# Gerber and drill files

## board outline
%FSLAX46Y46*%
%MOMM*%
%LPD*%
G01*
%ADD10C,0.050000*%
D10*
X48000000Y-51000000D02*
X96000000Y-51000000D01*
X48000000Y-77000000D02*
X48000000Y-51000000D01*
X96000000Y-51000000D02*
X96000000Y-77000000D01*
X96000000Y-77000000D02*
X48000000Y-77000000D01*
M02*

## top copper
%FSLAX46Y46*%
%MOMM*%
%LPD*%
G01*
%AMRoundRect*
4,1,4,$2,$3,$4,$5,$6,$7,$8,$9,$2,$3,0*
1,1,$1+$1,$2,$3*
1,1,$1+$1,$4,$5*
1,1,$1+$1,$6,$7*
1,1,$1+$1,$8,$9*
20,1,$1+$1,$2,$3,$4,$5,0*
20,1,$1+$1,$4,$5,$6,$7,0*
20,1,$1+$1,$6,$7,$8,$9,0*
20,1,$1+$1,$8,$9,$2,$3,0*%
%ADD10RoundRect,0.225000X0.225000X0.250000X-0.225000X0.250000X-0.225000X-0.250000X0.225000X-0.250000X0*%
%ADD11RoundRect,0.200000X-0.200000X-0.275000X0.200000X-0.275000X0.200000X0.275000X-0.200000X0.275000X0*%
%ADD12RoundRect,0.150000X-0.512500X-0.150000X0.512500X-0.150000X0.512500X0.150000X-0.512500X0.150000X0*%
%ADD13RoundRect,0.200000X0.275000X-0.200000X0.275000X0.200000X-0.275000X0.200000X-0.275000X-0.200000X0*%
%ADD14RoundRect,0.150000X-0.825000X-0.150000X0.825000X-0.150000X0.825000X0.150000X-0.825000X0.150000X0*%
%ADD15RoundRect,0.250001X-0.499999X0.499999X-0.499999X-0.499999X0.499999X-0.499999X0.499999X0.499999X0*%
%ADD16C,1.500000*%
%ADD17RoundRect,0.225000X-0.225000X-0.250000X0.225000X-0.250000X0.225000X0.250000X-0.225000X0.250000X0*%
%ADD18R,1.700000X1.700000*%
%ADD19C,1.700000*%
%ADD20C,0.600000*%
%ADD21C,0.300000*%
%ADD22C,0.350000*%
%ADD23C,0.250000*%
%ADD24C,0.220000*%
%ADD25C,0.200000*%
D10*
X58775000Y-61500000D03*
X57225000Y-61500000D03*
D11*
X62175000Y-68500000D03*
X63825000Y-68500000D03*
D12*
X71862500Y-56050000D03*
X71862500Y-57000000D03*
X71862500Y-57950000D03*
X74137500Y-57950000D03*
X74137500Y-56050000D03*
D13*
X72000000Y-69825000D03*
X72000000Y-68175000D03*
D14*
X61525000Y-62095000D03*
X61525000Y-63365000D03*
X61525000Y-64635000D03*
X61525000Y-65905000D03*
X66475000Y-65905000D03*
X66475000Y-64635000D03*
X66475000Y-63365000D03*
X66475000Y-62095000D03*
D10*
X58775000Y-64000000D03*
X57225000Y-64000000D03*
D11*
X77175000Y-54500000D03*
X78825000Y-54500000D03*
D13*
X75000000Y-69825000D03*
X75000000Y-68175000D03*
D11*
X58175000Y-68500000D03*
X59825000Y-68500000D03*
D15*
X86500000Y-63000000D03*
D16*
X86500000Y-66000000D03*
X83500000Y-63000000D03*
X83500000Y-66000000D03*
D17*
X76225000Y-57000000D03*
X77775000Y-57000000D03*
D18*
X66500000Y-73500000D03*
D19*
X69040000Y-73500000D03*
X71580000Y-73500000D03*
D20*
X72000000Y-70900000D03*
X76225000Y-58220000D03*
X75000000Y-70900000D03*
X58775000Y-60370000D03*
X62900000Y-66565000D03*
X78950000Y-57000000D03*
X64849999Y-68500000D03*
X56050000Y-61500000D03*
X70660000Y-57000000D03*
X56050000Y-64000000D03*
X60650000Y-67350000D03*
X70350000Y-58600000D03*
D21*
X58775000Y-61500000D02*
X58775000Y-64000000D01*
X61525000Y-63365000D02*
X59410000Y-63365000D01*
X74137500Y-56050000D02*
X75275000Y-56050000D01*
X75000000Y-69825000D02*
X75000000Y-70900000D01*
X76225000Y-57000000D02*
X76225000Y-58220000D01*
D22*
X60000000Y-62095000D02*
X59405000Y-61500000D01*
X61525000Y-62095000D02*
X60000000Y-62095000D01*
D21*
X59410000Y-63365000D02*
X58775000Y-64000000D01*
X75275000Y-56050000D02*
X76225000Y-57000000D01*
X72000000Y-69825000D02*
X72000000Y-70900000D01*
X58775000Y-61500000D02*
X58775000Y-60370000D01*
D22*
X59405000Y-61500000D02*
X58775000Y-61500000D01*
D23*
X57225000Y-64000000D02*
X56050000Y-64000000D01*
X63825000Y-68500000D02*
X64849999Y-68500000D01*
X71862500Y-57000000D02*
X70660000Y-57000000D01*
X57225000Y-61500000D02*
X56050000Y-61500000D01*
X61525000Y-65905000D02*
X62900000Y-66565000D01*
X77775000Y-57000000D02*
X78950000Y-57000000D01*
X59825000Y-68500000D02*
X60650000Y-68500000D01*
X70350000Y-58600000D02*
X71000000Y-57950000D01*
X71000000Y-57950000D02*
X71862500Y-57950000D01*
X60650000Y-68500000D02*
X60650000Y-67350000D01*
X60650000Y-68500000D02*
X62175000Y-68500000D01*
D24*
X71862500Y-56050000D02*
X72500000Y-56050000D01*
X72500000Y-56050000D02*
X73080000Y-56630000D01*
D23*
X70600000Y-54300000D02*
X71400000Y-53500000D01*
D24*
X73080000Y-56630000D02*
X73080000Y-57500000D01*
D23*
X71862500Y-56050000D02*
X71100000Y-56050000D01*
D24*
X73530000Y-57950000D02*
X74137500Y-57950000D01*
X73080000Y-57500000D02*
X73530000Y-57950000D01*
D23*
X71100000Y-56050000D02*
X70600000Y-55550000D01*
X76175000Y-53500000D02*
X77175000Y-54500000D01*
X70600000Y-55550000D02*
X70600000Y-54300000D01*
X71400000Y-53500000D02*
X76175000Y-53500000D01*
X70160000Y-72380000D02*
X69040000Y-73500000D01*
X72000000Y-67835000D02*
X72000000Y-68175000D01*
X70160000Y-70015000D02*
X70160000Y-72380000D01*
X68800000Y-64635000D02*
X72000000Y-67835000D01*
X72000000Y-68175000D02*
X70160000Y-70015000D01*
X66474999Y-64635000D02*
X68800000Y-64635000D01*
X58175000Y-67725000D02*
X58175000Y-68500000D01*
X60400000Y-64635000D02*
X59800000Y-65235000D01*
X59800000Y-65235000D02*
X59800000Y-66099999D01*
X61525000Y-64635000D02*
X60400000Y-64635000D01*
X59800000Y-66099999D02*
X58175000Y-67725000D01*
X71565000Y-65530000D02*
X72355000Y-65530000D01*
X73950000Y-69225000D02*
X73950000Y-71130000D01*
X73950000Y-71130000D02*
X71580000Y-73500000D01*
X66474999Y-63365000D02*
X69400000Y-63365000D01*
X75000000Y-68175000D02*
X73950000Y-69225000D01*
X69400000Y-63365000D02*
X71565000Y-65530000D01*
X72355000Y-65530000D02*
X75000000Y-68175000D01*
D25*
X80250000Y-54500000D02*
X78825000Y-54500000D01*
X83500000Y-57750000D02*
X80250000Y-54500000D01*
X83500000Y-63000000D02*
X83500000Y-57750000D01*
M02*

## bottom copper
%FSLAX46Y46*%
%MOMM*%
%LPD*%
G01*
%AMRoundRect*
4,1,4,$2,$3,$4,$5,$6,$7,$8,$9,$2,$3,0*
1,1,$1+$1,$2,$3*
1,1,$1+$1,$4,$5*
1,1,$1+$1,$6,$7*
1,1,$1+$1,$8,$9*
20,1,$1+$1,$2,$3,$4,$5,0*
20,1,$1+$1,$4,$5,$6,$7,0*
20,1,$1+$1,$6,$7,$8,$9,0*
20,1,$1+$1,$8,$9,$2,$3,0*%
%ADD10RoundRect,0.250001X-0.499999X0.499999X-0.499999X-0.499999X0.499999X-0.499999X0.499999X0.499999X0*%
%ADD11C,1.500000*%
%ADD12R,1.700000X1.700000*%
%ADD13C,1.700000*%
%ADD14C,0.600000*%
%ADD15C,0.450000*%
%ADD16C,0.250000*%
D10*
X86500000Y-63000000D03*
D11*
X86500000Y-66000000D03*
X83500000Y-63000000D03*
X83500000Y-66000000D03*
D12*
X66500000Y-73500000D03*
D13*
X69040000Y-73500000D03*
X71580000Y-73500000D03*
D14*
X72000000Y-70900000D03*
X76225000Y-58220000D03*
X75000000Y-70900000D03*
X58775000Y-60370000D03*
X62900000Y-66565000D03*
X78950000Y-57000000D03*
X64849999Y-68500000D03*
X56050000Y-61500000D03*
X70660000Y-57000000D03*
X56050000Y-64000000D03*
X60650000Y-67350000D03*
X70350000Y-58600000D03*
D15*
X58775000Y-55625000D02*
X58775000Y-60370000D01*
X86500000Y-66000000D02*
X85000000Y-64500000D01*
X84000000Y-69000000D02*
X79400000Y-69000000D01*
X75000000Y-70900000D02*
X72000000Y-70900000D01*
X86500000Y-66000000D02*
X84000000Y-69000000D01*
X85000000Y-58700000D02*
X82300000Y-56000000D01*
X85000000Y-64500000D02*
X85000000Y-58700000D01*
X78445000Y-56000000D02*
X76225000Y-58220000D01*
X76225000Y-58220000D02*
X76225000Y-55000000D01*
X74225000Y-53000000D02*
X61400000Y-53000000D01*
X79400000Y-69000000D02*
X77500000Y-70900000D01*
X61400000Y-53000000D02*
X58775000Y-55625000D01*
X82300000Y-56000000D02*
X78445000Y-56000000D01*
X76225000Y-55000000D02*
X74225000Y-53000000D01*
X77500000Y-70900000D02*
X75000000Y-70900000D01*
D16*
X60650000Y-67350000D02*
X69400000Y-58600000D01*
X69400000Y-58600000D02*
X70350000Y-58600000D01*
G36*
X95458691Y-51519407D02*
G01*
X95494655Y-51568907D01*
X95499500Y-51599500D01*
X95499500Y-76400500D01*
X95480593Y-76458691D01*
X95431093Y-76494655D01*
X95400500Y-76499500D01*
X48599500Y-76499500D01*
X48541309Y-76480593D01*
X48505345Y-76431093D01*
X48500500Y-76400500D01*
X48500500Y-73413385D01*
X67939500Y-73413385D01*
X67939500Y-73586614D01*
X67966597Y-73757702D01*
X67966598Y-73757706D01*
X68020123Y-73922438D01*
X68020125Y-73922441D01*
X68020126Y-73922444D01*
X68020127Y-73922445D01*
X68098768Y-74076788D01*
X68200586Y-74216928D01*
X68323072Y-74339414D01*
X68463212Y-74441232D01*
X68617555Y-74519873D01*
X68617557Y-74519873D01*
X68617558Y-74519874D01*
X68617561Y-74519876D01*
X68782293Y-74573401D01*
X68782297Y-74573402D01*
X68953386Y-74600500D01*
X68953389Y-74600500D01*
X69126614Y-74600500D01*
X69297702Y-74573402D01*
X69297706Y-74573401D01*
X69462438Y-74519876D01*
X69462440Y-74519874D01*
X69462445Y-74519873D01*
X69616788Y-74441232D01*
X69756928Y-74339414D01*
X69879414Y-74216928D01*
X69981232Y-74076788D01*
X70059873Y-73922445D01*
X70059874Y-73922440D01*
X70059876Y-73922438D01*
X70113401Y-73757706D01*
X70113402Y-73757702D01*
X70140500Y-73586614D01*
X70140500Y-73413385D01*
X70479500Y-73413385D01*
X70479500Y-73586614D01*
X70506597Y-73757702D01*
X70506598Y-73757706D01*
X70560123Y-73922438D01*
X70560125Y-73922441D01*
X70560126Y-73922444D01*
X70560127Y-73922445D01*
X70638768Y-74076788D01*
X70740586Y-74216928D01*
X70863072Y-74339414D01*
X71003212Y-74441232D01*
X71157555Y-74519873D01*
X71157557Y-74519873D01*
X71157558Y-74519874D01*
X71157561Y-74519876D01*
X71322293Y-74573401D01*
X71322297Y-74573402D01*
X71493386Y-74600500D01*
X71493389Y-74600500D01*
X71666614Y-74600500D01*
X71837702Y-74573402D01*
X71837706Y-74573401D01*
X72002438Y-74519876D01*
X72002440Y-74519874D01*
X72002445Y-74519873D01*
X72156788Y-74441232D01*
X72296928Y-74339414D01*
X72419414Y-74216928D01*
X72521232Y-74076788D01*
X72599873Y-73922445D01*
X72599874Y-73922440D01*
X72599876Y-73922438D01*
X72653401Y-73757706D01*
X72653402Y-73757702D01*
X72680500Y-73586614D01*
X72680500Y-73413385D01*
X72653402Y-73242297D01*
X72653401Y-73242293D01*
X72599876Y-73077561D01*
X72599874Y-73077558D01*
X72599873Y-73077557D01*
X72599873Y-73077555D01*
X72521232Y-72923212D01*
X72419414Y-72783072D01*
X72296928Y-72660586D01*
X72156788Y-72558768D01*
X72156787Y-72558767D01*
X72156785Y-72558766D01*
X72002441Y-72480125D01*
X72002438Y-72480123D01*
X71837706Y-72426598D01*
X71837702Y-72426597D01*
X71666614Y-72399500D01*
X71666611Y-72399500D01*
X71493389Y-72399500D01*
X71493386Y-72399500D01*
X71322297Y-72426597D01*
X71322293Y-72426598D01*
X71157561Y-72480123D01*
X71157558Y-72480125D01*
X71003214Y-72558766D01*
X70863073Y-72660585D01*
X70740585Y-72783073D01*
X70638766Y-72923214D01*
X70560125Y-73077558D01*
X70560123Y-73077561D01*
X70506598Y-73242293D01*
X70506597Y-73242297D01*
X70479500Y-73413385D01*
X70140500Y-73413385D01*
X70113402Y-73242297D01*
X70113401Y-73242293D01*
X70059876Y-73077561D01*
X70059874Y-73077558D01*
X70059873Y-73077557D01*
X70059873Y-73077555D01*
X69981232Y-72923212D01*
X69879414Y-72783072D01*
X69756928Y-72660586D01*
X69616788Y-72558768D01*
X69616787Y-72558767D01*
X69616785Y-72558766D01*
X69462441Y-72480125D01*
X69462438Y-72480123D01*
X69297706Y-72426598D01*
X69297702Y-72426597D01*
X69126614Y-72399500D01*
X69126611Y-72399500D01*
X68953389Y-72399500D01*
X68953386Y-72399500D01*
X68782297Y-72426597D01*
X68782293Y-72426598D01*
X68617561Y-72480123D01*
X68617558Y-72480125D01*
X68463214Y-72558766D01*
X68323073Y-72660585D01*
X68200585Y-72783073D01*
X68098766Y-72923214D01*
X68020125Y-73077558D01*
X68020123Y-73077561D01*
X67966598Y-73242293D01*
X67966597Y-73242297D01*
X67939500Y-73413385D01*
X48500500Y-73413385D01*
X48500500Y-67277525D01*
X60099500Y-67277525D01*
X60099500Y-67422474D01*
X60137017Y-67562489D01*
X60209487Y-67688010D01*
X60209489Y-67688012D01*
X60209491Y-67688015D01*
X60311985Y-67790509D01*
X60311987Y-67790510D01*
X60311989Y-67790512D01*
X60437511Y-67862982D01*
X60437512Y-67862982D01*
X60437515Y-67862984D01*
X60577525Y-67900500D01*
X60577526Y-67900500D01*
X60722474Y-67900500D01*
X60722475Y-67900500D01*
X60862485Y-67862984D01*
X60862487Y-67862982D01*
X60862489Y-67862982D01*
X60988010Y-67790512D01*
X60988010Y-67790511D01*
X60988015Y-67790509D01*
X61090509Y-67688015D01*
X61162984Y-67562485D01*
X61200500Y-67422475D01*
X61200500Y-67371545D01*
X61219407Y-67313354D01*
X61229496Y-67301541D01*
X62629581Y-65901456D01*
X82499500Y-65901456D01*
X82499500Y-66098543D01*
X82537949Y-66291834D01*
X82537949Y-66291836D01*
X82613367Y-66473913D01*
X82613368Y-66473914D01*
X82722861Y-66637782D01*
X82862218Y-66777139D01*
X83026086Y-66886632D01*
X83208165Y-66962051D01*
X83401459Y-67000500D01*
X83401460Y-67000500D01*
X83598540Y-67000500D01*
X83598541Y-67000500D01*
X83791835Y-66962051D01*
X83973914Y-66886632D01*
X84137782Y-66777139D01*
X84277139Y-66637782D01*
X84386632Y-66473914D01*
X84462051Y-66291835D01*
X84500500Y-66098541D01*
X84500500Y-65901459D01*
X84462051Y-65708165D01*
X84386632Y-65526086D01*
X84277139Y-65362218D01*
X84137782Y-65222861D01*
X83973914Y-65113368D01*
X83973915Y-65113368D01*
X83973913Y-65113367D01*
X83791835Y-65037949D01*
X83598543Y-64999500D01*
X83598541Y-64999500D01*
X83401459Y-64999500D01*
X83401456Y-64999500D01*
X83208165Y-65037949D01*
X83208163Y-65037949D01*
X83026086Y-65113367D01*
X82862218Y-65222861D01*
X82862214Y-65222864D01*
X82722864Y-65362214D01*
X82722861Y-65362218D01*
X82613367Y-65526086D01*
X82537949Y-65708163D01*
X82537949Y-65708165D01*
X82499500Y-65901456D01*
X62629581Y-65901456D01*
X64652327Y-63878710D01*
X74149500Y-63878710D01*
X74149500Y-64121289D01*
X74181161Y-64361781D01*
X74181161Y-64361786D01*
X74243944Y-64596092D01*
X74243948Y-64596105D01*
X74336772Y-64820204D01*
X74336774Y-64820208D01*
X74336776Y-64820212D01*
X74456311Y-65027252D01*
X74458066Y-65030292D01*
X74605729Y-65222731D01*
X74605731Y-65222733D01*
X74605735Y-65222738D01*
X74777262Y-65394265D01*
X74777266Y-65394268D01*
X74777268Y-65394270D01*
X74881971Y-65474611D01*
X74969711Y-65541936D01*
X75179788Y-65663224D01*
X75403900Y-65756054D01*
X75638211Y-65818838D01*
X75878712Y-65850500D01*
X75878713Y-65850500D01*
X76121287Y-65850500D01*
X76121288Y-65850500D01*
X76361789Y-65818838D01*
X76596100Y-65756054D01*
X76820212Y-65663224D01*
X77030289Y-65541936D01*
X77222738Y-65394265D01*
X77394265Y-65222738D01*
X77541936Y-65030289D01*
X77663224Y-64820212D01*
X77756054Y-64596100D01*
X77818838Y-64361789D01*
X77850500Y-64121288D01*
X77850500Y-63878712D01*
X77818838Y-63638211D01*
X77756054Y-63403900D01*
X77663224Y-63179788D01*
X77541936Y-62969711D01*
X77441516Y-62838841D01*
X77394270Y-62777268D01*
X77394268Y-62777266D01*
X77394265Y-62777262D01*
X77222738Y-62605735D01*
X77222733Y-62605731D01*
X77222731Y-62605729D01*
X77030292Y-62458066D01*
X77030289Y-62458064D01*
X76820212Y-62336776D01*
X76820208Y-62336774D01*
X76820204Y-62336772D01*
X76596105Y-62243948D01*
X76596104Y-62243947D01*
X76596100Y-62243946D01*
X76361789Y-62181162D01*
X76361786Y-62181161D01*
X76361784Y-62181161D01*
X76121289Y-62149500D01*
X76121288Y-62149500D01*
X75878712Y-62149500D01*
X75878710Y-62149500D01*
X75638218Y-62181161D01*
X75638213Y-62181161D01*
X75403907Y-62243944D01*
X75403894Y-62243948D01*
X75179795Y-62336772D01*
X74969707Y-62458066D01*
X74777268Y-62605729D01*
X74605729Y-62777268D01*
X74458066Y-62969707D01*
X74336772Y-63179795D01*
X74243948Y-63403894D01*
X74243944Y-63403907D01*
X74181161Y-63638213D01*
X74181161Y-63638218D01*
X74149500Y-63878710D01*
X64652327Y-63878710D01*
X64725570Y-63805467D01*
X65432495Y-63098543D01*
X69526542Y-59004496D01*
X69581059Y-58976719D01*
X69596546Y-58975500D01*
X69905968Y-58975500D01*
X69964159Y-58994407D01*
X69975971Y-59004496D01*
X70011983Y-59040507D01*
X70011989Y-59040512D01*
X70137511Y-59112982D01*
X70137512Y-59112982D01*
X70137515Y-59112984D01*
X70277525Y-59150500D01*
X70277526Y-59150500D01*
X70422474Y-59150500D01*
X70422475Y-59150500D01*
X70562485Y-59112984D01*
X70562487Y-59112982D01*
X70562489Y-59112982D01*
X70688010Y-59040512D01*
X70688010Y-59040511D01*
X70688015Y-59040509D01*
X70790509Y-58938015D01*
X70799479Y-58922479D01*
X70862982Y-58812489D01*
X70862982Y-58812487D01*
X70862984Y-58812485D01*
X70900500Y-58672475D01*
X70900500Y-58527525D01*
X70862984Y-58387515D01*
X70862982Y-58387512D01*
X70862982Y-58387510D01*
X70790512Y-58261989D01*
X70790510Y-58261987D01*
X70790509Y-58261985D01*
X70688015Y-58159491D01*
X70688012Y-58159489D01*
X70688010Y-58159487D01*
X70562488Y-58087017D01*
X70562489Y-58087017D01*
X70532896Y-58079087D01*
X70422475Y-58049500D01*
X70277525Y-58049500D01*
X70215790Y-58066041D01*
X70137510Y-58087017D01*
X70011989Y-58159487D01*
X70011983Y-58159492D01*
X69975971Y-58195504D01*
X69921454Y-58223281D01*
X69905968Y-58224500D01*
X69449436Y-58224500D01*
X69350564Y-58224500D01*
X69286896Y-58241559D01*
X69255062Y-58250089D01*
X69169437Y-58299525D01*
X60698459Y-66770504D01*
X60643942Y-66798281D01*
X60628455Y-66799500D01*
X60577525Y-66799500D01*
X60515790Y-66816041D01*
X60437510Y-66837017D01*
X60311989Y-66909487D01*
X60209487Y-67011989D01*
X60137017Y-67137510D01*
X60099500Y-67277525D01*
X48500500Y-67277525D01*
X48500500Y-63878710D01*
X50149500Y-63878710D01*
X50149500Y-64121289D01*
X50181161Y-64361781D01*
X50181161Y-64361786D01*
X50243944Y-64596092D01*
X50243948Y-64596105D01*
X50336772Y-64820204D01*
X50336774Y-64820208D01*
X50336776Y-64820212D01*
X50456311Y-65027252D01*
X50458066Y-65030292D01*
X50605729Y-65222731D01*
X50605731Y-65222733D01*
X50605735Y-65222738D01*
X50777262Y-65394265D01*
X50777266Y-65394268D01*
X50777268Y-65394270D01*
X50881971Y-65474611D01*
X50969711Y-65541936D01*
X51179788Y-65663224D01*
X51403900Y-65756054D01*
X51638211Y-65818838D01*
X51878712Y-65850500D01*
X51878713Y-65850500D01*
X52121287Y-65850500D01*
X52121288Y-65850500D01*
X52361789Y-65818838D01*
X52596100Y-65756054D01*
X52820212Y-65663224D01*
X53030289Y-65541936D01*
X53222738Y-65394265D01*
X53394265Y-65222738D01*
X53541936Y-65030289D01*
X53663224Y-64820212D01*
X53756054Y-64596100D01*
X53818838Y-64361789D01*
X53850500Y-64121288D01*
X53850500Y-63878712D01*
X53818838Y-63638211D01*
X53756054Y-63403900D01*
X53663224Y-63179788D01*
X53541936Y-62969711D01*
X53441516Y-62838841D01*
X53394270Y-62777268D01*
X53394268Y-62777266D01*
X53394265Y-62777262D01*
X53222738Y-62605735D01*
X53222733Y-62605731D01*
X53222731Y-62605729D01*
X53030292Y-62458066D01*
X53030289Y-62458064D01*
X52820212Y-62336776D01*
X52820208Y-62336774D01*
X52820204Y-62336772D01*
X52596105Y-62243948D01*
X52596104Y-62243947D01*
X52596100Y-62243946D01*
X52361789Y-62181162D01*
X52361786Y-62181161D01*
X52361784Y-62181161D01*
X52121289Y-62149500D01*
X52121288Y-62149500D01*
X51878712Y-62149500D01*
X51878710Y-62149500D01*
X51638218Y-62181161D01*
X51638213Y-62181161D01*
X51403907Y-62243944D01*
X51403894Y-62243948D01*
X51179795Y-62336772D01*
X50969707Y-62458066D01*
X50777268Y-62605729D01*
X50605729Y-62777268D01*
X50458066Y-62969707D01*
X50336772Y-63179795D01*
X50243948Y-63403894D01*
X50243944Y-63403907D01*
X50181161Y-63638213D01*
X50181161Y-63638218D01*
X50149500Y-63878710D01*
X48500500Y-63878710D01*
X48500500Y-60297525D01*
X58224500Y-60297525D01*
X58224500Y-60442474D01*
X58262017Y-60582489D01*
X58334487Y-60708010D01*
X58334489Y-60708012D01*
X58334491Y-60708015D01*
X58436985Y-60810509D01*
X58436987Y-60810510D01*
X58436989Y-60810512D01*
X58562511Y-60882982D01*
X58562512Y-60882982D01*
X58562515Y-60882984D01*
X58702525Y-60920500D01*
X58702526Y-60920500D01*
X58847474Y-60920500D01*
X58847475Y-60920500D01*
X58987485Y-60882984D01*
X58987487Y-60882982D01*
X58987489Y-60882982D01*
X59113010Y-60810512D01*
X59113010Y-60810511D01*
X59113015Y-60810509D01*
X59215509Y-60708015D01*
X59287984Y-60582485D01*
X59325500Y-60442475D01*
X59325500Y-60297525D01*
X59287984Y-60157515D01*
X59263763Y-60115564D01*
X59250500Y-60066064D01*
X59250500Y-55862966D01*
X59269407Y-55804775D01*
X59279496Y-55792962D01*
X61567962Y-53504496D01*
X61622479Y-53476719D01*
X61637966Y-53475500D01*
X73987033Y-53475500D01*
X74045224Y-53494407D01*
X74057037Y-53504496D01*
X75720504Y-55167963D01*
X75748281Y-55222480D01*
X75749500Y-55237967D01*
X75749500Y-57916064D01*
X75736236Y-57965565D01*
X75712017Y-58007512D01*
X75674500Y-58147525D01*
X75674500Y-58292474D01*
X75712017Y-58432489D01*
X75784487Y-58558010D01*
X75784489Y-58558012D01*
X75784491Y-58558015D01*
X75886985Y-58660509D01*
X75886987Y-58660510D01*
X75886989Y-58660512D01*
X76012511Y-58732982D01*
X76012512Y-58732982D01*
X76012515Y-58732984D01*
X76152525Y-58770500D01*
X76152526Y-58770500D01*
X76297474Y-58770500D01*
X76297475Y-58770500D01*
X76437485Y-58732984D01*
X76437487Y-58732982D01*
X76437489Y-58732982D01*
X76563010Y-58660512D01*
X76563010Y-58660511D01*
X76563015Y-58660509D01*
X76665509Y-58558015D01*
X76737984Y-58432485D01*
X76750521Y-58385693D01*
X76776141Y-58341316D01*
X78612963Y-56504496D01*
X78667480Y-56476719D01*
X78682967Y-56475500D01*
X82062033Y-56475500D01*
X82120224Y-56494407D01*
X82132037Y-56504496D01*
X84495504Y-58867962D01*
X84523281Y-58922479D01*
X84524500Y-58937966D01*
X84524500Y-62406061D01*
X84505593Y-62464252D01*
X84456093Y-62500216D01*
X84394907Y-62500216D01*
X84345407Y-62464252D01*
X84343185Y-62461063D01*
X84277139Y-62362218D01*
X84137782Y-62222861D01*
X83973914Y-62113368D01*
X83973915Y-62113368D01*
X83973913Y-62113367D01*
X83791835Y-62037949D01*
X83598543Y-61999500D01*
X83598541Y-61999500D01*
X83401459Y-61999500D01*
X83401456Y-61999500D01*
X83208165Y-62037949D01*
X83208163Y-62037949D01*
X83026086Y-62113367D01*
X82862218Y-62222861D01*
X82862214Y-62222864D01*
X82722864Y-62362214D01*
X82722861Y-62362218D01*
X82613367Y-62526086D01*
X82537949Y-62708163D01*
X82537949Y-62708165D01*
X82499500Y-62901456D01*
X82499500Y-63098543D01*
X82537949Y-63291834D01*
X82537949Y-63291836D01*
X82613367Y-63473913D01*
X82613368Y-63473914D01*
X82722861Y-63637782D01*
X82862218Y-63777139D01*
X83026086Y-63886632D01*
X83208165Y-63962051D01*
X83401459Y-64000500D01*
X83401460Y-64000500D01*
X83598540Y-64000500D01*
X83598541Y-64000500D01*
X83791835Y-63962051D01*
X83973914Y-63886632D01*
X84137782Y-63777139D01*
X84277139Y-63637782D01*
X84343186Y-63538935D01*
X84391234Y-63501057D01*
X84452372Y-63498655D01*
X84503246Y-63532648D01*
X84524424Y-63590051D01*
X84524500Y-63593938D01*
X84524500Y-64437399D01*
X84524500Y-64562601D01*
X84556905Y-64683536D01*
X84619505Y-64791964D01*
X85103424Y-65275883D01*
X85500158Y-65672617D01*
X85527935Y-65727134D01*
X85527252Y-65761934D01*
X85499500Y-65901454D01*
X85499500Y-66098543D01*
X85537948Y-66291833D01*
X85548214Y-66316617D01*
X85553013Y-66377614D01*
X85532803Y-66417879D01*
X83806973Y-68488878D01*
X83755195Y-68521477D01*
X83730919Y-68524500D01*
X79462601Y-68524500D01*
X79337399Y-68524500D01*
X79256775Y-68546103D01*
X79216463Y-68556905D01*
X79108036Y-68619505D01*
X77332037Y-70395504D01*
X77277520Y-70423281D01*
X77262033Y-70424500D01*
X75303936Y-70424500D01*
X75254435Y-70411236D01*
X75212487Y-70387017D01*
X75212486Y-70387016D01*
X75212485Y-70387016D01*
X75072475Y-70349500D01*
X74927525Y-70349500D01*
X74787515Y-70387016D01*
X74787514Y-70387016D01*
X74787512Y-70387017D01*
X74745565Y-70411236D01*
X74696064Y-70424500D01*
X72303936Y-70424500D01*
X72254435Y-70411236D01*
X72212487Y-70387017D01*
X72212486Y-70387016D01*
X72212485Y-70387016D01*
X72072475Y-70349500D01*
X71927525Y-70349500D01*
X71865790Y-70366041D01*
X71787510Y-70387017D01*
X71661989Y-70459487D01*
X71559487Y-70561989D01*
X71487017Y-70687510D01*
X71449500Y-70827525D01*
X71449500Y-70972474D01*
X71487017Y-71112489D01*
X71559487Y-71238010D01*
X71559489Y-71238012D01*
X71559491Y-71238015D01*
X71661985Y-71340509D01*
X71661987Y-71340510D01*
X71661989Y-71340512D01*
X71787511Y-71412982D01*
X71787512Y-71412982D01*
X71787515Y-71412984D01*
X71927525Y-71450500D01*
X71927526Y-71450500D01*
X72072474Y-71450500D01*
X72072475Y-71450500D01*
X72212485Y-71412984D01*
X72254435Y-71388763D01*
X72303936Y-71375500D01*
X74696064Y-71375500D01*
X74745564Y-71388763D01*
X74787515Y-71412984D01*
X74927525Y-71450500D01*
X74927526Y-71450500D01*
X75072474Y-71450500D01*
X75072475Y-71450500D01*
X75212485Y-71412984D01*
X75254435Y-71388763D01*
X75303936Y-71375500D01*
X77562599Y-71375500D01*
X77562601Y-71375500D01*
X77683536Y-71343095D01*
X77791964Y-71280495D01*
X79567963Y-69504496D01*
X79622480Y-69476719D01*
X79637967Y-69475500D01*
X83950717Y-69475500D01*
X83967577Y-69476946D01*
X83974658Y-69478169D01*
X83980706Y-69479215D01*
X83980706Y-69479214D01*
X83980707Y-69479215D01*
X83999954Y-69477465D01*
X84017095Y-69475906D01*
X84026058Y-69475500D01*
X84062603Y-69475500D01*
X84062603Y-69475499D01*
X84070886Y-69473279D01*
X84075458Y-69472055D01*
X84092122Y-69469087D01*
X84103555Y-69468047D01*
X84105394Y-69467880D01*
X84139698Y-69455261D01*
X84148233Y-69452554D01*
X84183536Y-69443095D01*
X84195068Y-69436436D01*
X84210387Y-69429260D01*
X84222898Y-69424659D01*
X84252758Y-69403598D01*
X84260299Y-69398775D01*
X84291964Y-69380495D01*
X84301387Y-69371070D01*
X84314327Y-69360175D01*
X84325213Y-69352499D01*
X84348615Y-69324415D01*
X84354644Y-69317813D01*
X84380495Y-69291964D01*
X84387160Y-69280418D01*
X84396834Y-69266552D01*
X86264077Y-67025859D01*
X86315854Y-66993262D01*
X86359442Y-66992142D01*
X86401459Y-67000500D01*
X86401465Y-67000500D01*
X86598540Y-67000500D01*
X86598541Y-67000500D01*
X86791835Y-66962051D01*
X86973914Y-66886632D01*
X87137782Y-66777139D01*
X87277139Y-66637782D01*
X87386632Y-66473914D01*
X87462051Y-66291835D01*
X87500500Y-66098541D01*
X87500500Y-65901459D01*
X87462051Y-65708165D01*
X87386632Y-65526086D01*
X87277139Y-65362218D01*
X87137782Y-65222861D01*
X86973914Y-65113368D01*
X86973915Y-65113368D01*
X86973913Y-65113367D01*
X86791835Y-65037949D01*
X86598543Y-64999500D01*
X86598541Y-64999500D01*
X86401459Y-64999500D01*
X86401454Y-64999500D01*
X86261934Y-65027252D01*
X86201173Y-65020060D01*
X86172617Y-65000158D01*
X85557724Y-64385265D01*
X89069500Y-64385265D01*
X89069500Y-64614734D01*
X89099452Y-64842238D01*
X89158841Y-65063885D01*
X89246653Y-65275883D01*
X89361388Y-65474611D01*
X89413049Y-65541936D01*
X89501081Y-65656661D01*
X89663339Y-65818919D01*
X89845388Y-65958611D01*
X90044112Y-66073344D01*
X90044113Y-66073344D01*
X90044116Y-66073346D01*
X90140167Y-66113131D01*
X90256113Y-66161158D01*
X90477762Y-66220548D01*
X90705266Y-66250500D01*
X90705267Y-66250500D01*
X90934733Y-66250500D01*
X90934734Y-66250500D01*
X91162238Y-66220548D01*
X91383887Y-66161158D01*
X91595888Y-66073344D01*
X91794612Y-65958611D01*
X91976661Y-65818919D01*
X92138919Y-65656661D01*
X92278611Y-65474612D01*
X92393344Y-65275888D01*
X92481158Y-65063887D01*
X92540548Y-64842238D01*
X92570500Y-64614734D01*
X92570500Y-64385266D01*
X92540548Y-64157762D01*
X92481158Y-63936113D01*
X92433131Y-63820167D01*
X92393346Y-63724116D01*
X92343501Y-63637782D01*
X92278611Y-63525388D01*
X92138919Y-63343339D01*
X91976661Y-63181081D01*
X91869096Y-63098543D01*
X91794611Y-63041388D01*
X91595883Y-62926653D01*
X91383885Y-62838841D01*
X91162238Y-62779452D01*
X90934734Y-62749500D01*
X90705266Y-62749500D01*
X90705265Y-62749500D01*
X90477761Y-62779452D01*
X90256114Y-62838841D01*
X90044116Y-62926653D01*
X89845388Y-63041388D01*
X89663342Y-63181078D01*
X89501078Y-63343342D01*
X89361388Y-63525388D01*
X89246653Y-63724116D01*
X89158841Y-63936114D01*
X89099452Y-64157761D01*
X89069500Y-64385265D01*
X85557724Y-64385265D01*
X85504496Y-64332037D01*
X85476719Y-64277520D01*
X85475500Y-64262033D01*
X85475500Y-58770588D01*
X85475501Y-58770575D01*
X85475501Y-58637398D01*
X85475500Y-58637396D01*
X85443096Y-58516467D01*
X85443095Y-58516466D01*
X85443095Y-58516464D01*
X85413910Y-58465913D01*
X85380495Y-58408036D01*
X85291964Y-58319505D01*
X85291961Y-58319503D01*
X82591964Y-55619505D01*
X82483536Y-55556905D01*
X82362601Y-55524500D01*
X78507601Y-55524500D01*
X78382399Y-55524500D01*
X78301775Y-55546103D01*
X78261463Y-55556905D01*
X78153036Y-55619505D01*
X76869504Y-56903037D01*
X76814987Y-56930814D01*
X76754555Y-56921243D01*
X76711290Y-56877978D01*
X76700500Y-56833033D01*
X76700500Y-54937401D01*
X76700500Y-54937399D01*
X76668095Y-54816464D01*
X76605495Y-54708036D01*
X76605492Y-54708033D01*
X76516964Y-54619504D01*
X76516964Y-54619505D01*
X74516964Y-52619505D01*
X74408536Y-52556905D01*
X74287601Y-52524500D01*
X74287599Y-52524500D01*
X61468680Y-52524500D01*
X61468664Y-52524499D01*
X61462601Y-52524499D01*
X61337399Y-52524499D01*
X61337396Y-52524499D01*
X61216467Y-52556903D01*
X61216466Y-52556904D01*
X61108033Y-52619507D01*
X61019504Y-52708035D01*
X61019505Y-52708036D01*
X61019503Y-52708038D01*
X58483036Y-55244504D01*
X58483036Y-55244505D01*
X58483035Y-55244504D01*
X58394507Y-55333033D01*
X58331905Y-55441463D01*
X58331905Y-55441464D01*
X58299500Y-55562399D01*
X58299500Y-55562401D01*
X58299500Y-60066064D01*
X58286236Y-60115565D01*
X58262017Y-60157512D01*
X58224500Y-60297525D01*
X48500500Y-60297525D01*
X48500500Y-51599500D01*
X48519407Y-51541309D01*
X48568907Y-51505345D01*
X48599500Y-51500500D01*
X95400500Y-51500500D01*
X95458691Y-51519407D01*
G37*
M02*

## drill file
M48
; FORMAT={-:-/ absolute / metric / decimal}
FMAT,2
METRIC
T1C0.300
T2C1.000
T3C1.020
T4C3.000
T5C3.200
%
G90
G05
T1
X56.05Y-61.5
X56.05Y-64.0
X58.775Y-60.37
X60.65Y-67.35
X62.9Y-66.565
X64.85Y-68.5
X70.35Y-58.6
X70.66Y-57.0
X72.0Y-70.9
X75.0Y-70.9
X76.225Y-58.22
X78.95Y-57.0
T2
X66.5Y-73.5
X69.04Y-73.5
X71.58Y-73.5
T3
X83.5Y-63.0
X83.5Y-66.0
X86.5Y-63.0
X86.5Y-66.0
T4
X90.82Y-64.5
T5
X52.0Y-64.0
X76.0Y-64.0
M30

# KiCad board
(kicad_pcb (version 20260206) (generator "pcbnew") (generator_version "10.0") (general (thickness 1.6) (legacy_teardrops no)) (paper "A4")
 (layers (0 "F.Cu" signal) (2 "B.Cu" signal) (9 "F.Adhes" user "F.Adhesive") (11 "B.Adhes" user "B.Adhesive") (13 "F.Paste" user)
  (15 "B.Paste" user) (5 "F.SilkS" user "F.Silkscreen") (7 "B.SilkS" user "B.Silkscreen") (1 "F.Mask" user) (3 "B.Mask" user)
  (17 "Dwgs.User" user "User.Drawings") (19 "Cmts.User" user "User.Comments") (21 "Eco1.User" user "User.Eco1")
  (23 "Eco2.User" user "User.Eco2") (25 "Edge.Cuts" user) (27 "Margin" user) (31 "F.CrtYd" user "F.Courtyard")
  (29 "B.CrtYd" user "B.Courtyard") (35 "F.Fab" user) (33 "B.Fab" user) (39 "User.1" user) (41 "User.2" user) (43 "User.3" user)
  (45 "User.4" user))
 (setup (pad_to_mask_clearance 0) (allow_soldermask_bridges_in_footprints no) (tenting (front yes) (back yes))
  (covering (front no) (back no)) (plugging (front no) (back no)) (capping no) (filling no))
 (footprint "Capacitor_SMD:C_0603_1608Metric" (layer "F.Cu") (at 58 61.5 180)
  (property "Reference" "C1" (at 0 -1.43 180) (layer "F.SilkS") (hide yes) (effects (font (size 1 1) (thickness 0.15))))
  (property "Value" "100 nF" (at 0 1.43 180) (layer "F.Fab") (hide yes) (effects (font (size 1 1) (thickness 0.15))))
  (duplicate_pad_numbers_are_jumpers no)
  (pad "1" smd roundrect (at -0.775 0 180) (size 0.9 0.95) (layers "F.Cu" "F.Mask" "F.Paste") (roundrect_rratio 0.25) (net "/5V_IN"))
  (pad "2" smd roundrect (at 0.775 0 180) (size 0.9 0.95) (layers "F.Cu" "F.Mask" "F.Paste") (roundrect_rratio 0.25) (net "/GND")))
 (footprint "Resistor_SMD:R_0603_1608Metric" (layer "F.Cu") (at 63 68.5)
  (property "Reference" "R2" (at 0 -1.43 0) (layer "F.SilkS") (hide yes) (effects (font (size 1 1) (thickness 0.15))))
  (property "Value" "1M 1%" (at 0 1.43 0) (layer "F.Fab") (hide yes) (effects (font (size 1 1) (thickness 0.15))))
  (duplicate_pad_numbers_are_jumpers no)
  (pad "1" smd roundrect (at -0.825 0) (size 0.8 0.95) (layers "F.Cu" "F.Mask" "F.Paste") (roundrect_rratio 0.25) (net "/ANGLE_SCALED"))
  (pad "2" smd roundrect (at 0.825 0) (size 0.8 0.95) (layers "F.Cu" "F.Mask" "F.Paste") (roundrect_rratio 0.25) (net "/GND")))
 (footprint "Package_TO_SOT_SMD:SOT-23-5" (layer "F.Cu") (at 73 57)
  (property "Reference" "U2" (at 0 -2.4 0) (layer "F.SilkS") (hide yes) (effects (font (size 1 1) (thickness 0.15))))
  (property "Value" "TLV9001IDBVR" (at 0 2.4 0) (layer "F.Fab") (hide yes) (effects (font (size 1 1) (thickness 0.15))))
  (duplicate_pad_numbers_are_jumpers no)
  (pad "1" smd roundrect (at -1.1375 -0.95) (size 1.325 0.6) (layers "F.Cu" "F.Mask" "F.Paste") (roundrect_rratio 0.25) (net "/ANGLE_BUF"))
  (pad "2" smd roundrect (at -1.1375 0) (size 1.325 0.6) (layers "F.Cu" "F.Mask" "F.Paste") (roundrect_rratio 0.25) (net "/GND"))
  (pad "3" smd roundrect (at -1.1375 0.95) (size 1.325 0.6) (layers "F.Cu" "F.Mask" "F.Paste") (roundrect_rratio 0.25) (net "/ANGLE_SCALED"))
  (pad "4" smd roundrect (at 1.1375 0.95) (size 1.325 0.6) (layers "F.Cu" "F.Mask" "F.Paste") (roundrect_rratio 0.25) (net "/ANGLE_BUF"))
  (pad "5" smd roundrect (at 1.1375 -0.95) (size 1.325 0.6) (layers "F.Cu" "F.Mask" "F.Paste") (roundrect_rratio 0.25) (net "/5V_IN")))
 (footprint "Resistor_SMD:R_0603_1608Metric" (layer "F.Cu") (at 72 69 90)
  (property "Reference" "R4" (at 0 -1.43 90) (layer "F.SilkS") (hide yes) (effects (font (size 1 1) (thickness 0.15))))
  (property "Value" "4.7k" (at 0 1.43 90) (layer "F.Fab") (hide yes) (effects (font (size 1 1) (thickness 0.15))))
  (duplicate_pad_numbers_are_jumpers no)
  (pad "1" smd roundrect (at -0.825 0 90) (size 0.8 0.95) (layers "F.Cu" "F.Mask" "F.Paste") (roundrect_rratio 0.25) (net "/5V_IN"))
  (pad "2" smd roundrect (at 0.825 0 90) (size 0.8 0.95) (layers "F.Cu" "F.Mask" "F.Paste") (roundrect_rratio 0.25) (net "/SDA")))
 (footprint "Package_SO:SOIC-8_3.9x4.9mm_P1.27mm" (layer "F.Cu") (at 64 64)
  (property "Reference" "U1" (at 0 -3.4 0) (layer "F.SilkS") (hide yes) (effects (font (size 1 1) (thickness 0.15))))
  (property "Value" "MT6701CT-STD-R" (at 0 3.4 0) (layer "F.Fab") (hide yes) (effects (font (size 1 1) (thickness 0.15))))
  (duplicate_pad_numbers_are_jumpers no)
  (pad "1" smd roundrect (at -2.475 -1.905) (size 1.95 0.6) (layers "F.Cu" "F.Mask" "F.Paste") (roundrect_rratio 0.25) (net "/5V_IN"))
  (pad "2" smd roundrect (at -2.475 -0.635) (size 1.95 0.6) (layers "F.Cu" "F.Mask" "F.Paste") (roundrect_rratio 0.25) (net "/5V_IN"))
  (pad "3" smd roundrect (at -2.475 0.635) (size 1.95 0.6) (layers "F.Cu" "F.Mask" "F.Paste") (roundrect_rratio 0.25) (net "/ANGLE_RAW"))
  (pad "4" smd roundrect (at -2.475 1.905) (size 1.95 0.6) (layers "F.Cu" "F.Mask" "F.Paste") (roundrect_rratio 0.25) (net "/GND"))
  (pad "5" smd roundrect (at 2.475 1.905) (size 1.95 0.6) (layers "F.Cu" "F.Mask" "F.Paste") (roundrect_rratio 0.25)
   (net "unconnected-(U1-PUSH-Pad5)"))
  (pad "6" smd roundrect (at 2.475 0.635) (size 1.95 0.6) (layers "F.Cu" "F.Mask" "F.Paste") (roundrect_rratio 0.25) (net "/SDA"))
  (pad "7" smd roundrect (at 2.475 -0.635) (size 1.95 0.6) (layers "F.Cu" "F.Mask" "F.Paste") (roundrect_rratio 0.25) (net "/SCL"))
  (pad "8" smd roundrect (at 2.475 -1.905) (size 1.95 0.6) (layers "F.Cu" "F.Mask" "F.Paste") (roundrect_rratio 0.25)
   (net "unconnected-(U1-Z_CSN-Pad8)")))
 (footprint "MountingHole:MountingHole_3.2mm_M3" (layer "F.Cu") (at 52 64)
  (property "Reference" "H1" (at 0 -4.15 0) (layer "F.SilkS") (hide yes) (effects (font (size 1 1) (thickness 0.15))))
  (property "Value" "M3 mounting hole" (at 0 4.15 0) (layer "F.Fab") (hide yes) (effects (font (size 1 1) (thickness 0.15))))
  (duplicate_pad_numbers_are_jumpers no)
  (pad "" np_thru_hole circle (at 0 0) (size 3.2 3.2) (drill 3.2) (layers "*.Cu" "*.Mask")))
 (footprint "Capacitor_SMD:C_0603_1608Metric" (layer "F.Cu") (at 58 64 180)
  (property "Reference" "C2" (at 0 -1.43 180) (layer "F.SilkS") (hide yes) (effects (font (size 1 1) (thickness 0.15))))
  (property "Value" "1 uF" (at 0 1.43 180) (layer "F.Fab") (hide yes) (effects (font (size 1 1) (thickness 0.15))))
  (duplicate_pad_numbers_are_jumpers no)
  (pad "1" smd roundrect (at -0.775 0 180) (size 0.9 0.95) (layers "F.Cu" "F.Mask" "F.Paste") (roundrect_rratio 0.25) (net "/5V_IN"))
  (pad "2" smd roundrect (at 0.775 0 180) (size 0.9 0.95) (layers "F.Cu" "F.Mask" "F.Paste") (roundrect_rratio 0.25) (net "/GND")))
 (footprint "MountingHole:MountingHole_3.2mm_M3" (layer "F.Cu") (at 76 64)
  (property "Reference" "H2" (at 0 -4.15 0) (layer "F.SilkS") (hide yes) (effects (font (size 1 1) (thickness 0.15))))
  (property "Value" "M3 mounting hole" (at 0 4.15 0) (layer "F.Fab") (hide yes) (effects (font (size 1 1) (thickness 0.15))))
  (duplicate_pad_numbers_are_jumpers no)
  (pad "" np_thru_hole circle (at 0 0) (size 3.2 3.2) (drill 3.2) (layers "*.Cu" "*.Mask")))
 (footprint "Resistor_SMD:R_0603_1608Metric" (layer "F.Cu") (at 78 54.5)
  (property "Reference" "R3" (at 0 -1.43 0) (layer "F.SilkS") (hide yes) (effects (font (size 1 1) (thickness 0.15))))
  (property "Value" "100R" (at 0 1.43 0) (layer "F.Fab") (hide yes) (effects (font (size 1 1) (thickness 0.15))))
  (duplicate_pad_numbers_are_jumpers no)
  (pad "1" smd roundrect (at -0.825 0) (size 0.8 0.95) (layers "F.Cu" "F.Mask" "F.Paste") (roundrect_rratio 0.25) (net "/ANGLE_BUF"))
  (pad "2" smd roundrect (at 0.825 0) (size 0.8 0.95) (layers "F.Cu" "F.Mask" "F.Paste") (roundrect_rratio 0.25) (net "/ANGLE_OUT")))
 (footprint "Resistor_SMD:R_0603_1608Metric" (layer "F.Cu") (at 75 69 90)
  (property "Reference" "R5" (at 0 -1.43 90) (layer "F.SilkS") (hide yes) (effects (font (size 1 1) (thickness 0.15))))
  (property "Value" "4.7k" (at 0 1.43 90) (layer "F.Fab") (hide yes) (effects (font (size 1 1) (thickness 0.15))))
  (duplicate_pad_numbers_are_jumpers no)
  (pad "1" smd roundrect (at -0.825 0 90) (size 0.8 0.95) (layers "F.Cu" "F.Mask" "F.Paste") (roundrect_rratio 0.25) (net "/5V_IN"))
  (pad "2" smd roundrect (at 0.825 0 90) (size 0.8 0.95) (layers "F.Cu" "F.Mask" "F.Paste") (roundrect_rratio 0.25) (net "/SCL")))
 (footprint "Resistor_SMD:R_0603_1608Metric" (layer "F.Cu") (at 59 68.5)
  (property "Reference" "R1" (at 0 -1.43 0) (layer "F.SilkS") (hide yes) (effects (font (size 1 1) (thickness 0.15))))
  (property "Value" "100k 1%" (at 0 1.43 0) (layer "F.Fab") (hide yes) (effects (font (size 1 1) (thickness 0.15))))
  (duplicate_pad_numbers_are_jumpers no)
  (pad "1" smd roundrect (at -0.825 0) (size 0.8 0.95) (layers "F.Cu" "F.Mask" "F.Paste") (roundrect_rratio 0.25) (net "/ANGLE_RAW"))
  (pad "2" smd roundrect (at 0.825 0) (size 0.8 0.95) (layers "F.Cu" "F.Mask" "F.Paste") (roundrect_rratio 0.25) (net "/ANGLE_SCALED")))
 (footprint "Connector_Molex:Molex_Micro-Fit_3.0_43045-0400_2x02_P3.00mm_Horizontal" (layer "F.Cu") (at 86.5 63 -90)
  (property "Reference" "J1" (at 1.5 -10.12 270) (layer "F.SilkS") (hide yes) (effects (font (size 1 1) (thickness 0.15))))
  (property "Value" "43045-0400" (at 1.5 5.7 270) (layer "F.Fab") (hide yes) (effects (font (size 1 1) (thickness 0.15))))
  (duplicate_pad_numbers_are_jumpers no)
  (pad "" np_thru_hole circle (at 1.5 -4.32 270) (size 3 3) (drill 3) (layers "*.Cu" "*.Mask"))
  (pad "1" thru_hole roundrect (at 0 0 270) (size 1.5 1.5) (drill 1.02) (layers "*.Cu" "*.Mask") (remove_unused_layers no)
   (roundrect_rratio 0.166667) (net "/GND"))
  (pad "2" thru_hole circle (at 3 0 270) (size 1.5 1.5) (drill 1.02) (layers "*.Cu" "*.Mask") (remove_unused_layers no) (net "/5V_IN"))
  (pad "3" thru_hole circle (at 0 3 270) (size 1.5 1.5) (drill 1.02) (layers "*.Cu" "*.Mask") (remove_unused_layers no) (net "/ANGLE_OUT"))
  (pad "4" thru_hole circle (at 3 3 270) (size 1.5 1.5) (drill 1.02) (layers "*.Cu" "*.Mask") (remove_unused_layers no)
   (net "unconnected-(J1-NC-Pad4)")))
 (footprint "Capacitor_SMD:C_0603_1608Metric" (layer "F.Cu") (at 77 57)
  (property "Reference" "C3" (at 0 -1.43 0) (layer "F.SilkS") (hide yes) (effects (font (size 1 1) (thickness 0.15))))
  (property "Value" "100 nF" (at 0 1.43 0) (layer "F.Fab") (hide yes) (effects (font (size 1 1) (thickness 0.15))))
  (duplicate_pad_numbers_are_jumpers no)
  (pad "1" smd roundrect (at -0.775 0) (size 0.9 0.95) (layers "F.Cu" "F.Mask" "F.Paste") (roundrect_rratio 0.25) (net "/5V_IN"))
  (pad "2" smd roundrect (at 0.775 0) (size 0.9 0.95) (layers "F.Cu" "F.Mask" "F.Paste") (roundrect_rratio 0.25) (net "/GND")))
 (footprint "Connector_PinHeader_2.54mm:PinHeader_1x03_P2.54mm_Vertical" (layer "F.Cu") (at 66.5 73.5 90)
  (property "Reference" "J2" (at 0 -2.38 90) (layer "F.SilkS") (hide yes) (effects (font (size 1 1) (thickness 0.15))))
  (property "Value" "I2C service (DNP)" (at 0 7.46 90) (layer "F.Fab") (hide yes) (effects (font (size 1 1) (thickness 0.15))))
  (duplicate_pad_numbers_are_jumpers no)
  (pad "1" thru_hole rect (at 0 0 90) (size 1.7 1.7) (drill 1) (layers "*.Cu" "*.Mask") (remove_unused_layers no) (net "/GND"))
  (pad "2" thru_hole circle (at 0 2.54 90) (size 1.7 1.7) (drill 1) (layers "*.Cu" "*.Mask") (remove_unused_layers no) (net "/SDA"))
  (pad "3" thru_hole circle (at 0 5.08 90) (size 1.7 1.7) (drill 1) (layers "*.Cu" "*.Mask") (remove_unused_layers no) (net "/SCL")))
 (gr_line (start 48 51) (end 96 51) (stroke (width 0.05) (type default)) (layer "Edge.Cuts"))
 (gr_line (start 48 77) (end 48 51) (stroke (width 0.05) (type default)) (layer "Edge.Cuts"))
 (gr_line (start 96 51) (end 96 77) (stroke (width 0.05) (type default)) (layer "Edge.Cuts"))
 (gr_line (start 96 77) (end 48 77) (stroke (width 0.05) (type default)) (layer "Edge.Cuts"))
 (segment (start 58.775 61.5) (end 58.775 64) (width 0.3) (layer "F.Cu") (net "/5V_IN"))
 (segment (start 61.525 63.365) (end 59.41 63.365) (width 0.3) (layer "F.Cu") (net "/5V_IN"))
 (segment (start 74.1375 56.05) (end 75.275 56.05) (width 0.3) (layer "F.Cu") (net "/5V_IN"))
 (segment (start 75 69.825) (end 75 70.9) (width 0.3) (layer "F.Cu") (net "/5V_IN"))
 (segment (start 76.225 57) (end 76.225 58.22) (width 0.3) (layer "F.Cu") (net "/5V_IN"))
 (segment (start 60 62.095) (end 59.405 61.5) (width 0.35) (layer "F.Cu") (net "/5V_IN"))
 (segment (start 61.525 62.095) (end 60 62.095) (width 0.35) (layer "F.Cu") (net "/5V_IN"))
 (segment (start 59.41 63.365) (end 58.775 64) (width 0.3) (layer "F.Cu") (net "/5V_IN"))
 (segment (start 75.275 56.05) (end 76.225 57) (width 0.3) (layer "F.Cu") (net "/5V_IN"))
 (segment (start 72 69.825) (end 72 70.9) (width 0.3) (layer "F.Cu") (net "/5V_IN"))
 (segment (start 58.775 61.5) (end 58.775 60.37) (width 0.3) (layer "F.Cu") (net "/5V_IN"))
 (segment (start 59.405 61.5) (end 58.775 61.5) (width 0.35) (layer "F.Cu") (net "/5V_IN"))
 (via (at 72 70.9) (size 0.6) (drill 0.3) (layers "F.Cu" "B.Cu") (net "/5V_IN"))
 (via (at 76.225 58.22) (size 0.6) (drill 0.3) (layers "F.Cu" "B.Cu") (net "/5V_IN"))
 (via (at 75 70.9) (size 0.6) (drill 0.3) (layers "F.Cu" "B.Cu") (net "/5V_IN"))
 (via (at 58.775 60.37) (size 0.6) (drill 0.3) (layers "F.Cu" "B.Cu") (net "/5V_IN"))
 (segment (start 58.775 55.625) (end 58.775 60.37) (width 0.45) (layer "B.Cu") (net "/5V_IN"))
 (segment (start 86.5 66) (end 85 64.5) (width 0.45) (layer "B.Cu") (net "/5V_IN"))
 (segment (start 84 69) (end 79.4 69) (width 0.45) (layer "B.Cu") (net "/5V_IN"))
 (segment (start 75 70.9) (end 72 70.9) (width 0.45) (layer "B.Cu") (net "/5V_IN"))
 (segment (start 86.5 66) (end 84 69) (width 0.45) (layer "B.Cu") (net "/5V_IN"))
 (segment (start 85 58.7) (end 82.3 56) (width 0.45) (layer "B.Cu") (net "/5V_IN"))
 (segment (start 85 64.5) (end 85 58.7) (width 0.45) (layer "B.Cu") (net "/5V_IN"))
 (segment (start 78.445 56) (end 76.225 58.22) (width 0.45) (layer "B.Cu") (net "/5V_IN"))
 (segment (start 76.225 58.22) (end 76.225 55) (width 0.45) (layer "B.Cu") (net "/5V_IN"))
 (segment (start 74.225 53) (end 61.4 53) (width 0.45) (layer "B.Cu") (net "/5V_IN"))
 (segment (start 79.4 69) (end 77.5 70.9) (width 0.45) (layer "B.Cu") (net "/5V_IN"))
 (segment (start 61.4 53) (end 58.775 55.625) (width 0.45) (layer "B.Cu") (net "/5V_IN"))
 (segment (start 82.3 56) (end 78.445 56) (width 0.45) (layer "B.Cu") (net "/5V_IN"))
 (segment (start 76.225 55) (end 74.225 53) (width 0.45) (layer "B.Cu") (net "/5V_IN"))
 (segment (start 77.5 70.9) (end 75 70.9) (width 0.45) (layer "B.Cu") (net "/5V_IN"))
 (segment (start 57.225 64) (end 56.05 64) (width 0.25) (layer "F.Cu") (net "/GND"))
 (segment (start 63.825 68.5) (end 64.849999 68.5) (width 0.25) (layer "F.Cu") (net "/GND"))
 (segment (start 71.8625 57) (end 70.66 57) (width 0.25) (layer "F.Cu") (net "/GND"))
 (segment (start 57.225 61.5) (end 56.05 61.5) (width 0.25) (layer "F.Cu") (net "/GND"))
 (segment (start 61.525 65.905) (end 62.9 66.565) (width 0.25) (layer "F.Cu") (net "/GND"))
 (segment (start 77.775 57) (end 78.95 57) (width 0.25) (layer "F.Cu") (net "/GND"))
 (via (at 62.9 66.565) (size 0.6) (drill 0.3) (layers "F.Cu" "B.Cu") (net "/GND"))
 (via (at 78.95 57) (size 0.6) (drill 0.3) (layers "F.Cu" "B.Cu") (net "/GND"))
 (via (at 64.849999 68.5) (size 0.6) (drill 0.3) (layers "F.Cu" "B.Cu") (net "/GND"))
 (via (at 56.05 61.5) (size 0.6) (drill 0.3) (layers "F.Cu" "B.Cu") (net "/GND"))
 (via (at 70.66 57) (size 0.6) (drill 0.3) (layers "F.Cu" "B.Cu") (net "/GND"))
 (via (at 56.05 64) (size 0.6) (drill 0.3) (layers "F.Cu" "B.Cu") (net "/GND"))
 (segment (start 59.825 68.5) (end 60.65 68.5) (width 0.25) (layer "F.Cu") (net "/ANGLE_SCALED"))
 (segment (start 70.35 58.6) (end 71 57.95) (width 0.25) (layer "F.Cu") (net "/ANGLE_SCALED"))
 (segment (start 71 57.95) (end 71.8625 57.95) (width 0.25) (layer "F.Cu") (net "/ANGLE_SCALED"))
 (segment (start 60.65 68.5) (end 60.65 67.35) (width 0.25) (layer "F.Cu") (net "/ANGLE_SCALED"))
 (segment (start 60.65 68.5) (end 62.175 68.5) (width 0.25) (layer "F.Cu") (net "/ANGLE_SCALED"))
 (via (at 60.65 67.35) (size 0.6) (drill 0.3) (layers "F.Cu" "B.Cu") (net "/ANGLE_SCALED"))
 (via (at 70.35 58.6) (size 0.6) (drill 0.3) (layers "F.Cu" "B.Cu") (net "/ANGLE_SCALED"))
 (segment (start 60.65 67.35) (end 69.4 58.6) (width 0.25) (layer "B.Cu") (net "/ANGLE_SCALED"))
 (segment (start 69.4 58.6) (end 70.35 58.6) (width 0.25) (layer "B.Cu") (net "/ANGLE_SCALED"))
 (segment (start 71.8625 56.05) (end 72.5 56.05) (width 0.22) (layer "F.Cu") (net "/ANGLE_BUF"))
 (segment (start 72.5 56.05) (end 73.08 56.63) (width 0.22) (layer "F.Cu") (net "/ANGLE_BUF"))
 (segment (start 70.6 54.3) (end 71.4 53.5) (width 0.25) (layer "F.Cu") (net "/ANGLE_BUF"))
 (segment (start 73.08 56.63) (end 73.08 57.5) (width 0.22) (layer "F.Cu") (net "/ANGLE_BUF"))
 (segment (start 71.8625 56.05) (end 71.1 56.05) (width 0.25) (layer "F.Cu") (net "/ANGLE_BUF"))
 (segment (start 73.53 57.95) (end 74.1375 57.95) (width 0.22) (layer "F.Cu") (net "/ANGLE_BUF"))
 (segment (start 73.08 57.5) (end 73.53 57.95) (width 0.22) (layer "F.Cu") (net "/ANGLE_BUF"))
 (segment (start 71.1 56.05) (end 70.6 55.55) (width 0.25) (layer "F.Cu") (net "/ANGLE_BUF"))
 (segment (start 76.175 53.5) (end 77.175 54.5) (width 0.25) (layer "F.Cu") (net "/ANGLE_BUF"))
 (segment (start 70.6 55.55) (end 70.6 54.3) (width 0.25) (layer "F.Cu") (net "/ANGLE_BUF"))
 (segment (start 71.4 53.5) (end 76.175 53.5) (width 0.25) (layer "F.Cu") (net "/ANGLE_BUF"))
 (segment (start 70.16 72.38) (end 69.04 73.5) (width 0.25) (layer "F.Cu") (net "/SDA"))
 (segment (start 72 67.835) (end 72 68.175) (width 0.25) (layer "F.Cu") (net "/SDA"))
 (segment (start 70.16 70.015) (end 70.16 72.38) (width 0.25) (layer "F.Cu") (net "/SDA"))
 (segment (start 68.8 64.635) (end 72 67.835) (width 0.25) (layer "F.Cu") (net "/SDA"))
 (segment (start 72 68.175) (end 70.16 70.015) (width 0.25) (layer "F.Cu") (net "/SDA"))
 (segment (start 66.474999 64.635) (end 68.8 64.635) (width 0.25) (layer "F.Cu") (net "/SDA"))
 (segment (start 58.175 67.725) (end 58.175 68.5) (width 0.25) (layer "F.Cu") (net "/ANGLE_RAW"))
 (segment (start 60.4 64.635) (end 59.8 65.235) (width 0.25) (layer "F.Cu") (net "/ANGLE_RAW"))
 (segment (start 59.8 65.235) (end 59.8 66.099999) (width 0.25) (layer "F.Cu") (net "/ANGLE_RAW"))
 (segment (start 61.525 64.635) (end 60.4 64.635) (width 0.25) (layer "F.Cu") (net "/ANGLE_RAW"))
 (segment (start 59.8 66.099999) (end 58.175 67.725) (width 0.25) (layer "F.Cu") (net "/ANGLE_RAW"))
 (segment (start 71.565 65.53) (end 72.355 65.53) (width 0.25) (layer "F.Cu") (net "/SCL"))
 (segment (start 73.95 69.225) (end 73.95 71.13) (width 0.25) (layer "F.Cu") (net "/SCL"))
 (segment (start 73.95 71.13) (end 71.58 73.5) (width 0.25) (layer "F.Cu") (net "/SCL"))
 (segment (start 66.474999 63.365) (end 69.4 63.365) (width 0.25) (layer "F.Cu") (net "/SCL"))
 (segment (start 75 68.175) (end 73.95 69.225) (width 0.25) (layer "F.Cu") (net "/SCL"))
 (segment (start 69.4 63.365) (end 71.565 65.53) (width 0.25) (layer "F.Cu") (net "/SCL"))
 (segment (start 72.355 65.53) (end 75 68.175) (width 0.25) (layer "F.Cu") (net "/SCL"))
 (segment (start 80.25 54.5) (end 78.825 54.5) (width 0.2) (layer "F.Cu") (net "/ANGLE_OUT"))
 (segment (start 83.5 57.75) (end 80.25 54.5) (width 0.2) (layer "F.Cu") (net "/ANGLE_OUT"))
 (segment (start 83.5 63) (end 83.5 57.75) (width 0.2) (layer "F.Cu") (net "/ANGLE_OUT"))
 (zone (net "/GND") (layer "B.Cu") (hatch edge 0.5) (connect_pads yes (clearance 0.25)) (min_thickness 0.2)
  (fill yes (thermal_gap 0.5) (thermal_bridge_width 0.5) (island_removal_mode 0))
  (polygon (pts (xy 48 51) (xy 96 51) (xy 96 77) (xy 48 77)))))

